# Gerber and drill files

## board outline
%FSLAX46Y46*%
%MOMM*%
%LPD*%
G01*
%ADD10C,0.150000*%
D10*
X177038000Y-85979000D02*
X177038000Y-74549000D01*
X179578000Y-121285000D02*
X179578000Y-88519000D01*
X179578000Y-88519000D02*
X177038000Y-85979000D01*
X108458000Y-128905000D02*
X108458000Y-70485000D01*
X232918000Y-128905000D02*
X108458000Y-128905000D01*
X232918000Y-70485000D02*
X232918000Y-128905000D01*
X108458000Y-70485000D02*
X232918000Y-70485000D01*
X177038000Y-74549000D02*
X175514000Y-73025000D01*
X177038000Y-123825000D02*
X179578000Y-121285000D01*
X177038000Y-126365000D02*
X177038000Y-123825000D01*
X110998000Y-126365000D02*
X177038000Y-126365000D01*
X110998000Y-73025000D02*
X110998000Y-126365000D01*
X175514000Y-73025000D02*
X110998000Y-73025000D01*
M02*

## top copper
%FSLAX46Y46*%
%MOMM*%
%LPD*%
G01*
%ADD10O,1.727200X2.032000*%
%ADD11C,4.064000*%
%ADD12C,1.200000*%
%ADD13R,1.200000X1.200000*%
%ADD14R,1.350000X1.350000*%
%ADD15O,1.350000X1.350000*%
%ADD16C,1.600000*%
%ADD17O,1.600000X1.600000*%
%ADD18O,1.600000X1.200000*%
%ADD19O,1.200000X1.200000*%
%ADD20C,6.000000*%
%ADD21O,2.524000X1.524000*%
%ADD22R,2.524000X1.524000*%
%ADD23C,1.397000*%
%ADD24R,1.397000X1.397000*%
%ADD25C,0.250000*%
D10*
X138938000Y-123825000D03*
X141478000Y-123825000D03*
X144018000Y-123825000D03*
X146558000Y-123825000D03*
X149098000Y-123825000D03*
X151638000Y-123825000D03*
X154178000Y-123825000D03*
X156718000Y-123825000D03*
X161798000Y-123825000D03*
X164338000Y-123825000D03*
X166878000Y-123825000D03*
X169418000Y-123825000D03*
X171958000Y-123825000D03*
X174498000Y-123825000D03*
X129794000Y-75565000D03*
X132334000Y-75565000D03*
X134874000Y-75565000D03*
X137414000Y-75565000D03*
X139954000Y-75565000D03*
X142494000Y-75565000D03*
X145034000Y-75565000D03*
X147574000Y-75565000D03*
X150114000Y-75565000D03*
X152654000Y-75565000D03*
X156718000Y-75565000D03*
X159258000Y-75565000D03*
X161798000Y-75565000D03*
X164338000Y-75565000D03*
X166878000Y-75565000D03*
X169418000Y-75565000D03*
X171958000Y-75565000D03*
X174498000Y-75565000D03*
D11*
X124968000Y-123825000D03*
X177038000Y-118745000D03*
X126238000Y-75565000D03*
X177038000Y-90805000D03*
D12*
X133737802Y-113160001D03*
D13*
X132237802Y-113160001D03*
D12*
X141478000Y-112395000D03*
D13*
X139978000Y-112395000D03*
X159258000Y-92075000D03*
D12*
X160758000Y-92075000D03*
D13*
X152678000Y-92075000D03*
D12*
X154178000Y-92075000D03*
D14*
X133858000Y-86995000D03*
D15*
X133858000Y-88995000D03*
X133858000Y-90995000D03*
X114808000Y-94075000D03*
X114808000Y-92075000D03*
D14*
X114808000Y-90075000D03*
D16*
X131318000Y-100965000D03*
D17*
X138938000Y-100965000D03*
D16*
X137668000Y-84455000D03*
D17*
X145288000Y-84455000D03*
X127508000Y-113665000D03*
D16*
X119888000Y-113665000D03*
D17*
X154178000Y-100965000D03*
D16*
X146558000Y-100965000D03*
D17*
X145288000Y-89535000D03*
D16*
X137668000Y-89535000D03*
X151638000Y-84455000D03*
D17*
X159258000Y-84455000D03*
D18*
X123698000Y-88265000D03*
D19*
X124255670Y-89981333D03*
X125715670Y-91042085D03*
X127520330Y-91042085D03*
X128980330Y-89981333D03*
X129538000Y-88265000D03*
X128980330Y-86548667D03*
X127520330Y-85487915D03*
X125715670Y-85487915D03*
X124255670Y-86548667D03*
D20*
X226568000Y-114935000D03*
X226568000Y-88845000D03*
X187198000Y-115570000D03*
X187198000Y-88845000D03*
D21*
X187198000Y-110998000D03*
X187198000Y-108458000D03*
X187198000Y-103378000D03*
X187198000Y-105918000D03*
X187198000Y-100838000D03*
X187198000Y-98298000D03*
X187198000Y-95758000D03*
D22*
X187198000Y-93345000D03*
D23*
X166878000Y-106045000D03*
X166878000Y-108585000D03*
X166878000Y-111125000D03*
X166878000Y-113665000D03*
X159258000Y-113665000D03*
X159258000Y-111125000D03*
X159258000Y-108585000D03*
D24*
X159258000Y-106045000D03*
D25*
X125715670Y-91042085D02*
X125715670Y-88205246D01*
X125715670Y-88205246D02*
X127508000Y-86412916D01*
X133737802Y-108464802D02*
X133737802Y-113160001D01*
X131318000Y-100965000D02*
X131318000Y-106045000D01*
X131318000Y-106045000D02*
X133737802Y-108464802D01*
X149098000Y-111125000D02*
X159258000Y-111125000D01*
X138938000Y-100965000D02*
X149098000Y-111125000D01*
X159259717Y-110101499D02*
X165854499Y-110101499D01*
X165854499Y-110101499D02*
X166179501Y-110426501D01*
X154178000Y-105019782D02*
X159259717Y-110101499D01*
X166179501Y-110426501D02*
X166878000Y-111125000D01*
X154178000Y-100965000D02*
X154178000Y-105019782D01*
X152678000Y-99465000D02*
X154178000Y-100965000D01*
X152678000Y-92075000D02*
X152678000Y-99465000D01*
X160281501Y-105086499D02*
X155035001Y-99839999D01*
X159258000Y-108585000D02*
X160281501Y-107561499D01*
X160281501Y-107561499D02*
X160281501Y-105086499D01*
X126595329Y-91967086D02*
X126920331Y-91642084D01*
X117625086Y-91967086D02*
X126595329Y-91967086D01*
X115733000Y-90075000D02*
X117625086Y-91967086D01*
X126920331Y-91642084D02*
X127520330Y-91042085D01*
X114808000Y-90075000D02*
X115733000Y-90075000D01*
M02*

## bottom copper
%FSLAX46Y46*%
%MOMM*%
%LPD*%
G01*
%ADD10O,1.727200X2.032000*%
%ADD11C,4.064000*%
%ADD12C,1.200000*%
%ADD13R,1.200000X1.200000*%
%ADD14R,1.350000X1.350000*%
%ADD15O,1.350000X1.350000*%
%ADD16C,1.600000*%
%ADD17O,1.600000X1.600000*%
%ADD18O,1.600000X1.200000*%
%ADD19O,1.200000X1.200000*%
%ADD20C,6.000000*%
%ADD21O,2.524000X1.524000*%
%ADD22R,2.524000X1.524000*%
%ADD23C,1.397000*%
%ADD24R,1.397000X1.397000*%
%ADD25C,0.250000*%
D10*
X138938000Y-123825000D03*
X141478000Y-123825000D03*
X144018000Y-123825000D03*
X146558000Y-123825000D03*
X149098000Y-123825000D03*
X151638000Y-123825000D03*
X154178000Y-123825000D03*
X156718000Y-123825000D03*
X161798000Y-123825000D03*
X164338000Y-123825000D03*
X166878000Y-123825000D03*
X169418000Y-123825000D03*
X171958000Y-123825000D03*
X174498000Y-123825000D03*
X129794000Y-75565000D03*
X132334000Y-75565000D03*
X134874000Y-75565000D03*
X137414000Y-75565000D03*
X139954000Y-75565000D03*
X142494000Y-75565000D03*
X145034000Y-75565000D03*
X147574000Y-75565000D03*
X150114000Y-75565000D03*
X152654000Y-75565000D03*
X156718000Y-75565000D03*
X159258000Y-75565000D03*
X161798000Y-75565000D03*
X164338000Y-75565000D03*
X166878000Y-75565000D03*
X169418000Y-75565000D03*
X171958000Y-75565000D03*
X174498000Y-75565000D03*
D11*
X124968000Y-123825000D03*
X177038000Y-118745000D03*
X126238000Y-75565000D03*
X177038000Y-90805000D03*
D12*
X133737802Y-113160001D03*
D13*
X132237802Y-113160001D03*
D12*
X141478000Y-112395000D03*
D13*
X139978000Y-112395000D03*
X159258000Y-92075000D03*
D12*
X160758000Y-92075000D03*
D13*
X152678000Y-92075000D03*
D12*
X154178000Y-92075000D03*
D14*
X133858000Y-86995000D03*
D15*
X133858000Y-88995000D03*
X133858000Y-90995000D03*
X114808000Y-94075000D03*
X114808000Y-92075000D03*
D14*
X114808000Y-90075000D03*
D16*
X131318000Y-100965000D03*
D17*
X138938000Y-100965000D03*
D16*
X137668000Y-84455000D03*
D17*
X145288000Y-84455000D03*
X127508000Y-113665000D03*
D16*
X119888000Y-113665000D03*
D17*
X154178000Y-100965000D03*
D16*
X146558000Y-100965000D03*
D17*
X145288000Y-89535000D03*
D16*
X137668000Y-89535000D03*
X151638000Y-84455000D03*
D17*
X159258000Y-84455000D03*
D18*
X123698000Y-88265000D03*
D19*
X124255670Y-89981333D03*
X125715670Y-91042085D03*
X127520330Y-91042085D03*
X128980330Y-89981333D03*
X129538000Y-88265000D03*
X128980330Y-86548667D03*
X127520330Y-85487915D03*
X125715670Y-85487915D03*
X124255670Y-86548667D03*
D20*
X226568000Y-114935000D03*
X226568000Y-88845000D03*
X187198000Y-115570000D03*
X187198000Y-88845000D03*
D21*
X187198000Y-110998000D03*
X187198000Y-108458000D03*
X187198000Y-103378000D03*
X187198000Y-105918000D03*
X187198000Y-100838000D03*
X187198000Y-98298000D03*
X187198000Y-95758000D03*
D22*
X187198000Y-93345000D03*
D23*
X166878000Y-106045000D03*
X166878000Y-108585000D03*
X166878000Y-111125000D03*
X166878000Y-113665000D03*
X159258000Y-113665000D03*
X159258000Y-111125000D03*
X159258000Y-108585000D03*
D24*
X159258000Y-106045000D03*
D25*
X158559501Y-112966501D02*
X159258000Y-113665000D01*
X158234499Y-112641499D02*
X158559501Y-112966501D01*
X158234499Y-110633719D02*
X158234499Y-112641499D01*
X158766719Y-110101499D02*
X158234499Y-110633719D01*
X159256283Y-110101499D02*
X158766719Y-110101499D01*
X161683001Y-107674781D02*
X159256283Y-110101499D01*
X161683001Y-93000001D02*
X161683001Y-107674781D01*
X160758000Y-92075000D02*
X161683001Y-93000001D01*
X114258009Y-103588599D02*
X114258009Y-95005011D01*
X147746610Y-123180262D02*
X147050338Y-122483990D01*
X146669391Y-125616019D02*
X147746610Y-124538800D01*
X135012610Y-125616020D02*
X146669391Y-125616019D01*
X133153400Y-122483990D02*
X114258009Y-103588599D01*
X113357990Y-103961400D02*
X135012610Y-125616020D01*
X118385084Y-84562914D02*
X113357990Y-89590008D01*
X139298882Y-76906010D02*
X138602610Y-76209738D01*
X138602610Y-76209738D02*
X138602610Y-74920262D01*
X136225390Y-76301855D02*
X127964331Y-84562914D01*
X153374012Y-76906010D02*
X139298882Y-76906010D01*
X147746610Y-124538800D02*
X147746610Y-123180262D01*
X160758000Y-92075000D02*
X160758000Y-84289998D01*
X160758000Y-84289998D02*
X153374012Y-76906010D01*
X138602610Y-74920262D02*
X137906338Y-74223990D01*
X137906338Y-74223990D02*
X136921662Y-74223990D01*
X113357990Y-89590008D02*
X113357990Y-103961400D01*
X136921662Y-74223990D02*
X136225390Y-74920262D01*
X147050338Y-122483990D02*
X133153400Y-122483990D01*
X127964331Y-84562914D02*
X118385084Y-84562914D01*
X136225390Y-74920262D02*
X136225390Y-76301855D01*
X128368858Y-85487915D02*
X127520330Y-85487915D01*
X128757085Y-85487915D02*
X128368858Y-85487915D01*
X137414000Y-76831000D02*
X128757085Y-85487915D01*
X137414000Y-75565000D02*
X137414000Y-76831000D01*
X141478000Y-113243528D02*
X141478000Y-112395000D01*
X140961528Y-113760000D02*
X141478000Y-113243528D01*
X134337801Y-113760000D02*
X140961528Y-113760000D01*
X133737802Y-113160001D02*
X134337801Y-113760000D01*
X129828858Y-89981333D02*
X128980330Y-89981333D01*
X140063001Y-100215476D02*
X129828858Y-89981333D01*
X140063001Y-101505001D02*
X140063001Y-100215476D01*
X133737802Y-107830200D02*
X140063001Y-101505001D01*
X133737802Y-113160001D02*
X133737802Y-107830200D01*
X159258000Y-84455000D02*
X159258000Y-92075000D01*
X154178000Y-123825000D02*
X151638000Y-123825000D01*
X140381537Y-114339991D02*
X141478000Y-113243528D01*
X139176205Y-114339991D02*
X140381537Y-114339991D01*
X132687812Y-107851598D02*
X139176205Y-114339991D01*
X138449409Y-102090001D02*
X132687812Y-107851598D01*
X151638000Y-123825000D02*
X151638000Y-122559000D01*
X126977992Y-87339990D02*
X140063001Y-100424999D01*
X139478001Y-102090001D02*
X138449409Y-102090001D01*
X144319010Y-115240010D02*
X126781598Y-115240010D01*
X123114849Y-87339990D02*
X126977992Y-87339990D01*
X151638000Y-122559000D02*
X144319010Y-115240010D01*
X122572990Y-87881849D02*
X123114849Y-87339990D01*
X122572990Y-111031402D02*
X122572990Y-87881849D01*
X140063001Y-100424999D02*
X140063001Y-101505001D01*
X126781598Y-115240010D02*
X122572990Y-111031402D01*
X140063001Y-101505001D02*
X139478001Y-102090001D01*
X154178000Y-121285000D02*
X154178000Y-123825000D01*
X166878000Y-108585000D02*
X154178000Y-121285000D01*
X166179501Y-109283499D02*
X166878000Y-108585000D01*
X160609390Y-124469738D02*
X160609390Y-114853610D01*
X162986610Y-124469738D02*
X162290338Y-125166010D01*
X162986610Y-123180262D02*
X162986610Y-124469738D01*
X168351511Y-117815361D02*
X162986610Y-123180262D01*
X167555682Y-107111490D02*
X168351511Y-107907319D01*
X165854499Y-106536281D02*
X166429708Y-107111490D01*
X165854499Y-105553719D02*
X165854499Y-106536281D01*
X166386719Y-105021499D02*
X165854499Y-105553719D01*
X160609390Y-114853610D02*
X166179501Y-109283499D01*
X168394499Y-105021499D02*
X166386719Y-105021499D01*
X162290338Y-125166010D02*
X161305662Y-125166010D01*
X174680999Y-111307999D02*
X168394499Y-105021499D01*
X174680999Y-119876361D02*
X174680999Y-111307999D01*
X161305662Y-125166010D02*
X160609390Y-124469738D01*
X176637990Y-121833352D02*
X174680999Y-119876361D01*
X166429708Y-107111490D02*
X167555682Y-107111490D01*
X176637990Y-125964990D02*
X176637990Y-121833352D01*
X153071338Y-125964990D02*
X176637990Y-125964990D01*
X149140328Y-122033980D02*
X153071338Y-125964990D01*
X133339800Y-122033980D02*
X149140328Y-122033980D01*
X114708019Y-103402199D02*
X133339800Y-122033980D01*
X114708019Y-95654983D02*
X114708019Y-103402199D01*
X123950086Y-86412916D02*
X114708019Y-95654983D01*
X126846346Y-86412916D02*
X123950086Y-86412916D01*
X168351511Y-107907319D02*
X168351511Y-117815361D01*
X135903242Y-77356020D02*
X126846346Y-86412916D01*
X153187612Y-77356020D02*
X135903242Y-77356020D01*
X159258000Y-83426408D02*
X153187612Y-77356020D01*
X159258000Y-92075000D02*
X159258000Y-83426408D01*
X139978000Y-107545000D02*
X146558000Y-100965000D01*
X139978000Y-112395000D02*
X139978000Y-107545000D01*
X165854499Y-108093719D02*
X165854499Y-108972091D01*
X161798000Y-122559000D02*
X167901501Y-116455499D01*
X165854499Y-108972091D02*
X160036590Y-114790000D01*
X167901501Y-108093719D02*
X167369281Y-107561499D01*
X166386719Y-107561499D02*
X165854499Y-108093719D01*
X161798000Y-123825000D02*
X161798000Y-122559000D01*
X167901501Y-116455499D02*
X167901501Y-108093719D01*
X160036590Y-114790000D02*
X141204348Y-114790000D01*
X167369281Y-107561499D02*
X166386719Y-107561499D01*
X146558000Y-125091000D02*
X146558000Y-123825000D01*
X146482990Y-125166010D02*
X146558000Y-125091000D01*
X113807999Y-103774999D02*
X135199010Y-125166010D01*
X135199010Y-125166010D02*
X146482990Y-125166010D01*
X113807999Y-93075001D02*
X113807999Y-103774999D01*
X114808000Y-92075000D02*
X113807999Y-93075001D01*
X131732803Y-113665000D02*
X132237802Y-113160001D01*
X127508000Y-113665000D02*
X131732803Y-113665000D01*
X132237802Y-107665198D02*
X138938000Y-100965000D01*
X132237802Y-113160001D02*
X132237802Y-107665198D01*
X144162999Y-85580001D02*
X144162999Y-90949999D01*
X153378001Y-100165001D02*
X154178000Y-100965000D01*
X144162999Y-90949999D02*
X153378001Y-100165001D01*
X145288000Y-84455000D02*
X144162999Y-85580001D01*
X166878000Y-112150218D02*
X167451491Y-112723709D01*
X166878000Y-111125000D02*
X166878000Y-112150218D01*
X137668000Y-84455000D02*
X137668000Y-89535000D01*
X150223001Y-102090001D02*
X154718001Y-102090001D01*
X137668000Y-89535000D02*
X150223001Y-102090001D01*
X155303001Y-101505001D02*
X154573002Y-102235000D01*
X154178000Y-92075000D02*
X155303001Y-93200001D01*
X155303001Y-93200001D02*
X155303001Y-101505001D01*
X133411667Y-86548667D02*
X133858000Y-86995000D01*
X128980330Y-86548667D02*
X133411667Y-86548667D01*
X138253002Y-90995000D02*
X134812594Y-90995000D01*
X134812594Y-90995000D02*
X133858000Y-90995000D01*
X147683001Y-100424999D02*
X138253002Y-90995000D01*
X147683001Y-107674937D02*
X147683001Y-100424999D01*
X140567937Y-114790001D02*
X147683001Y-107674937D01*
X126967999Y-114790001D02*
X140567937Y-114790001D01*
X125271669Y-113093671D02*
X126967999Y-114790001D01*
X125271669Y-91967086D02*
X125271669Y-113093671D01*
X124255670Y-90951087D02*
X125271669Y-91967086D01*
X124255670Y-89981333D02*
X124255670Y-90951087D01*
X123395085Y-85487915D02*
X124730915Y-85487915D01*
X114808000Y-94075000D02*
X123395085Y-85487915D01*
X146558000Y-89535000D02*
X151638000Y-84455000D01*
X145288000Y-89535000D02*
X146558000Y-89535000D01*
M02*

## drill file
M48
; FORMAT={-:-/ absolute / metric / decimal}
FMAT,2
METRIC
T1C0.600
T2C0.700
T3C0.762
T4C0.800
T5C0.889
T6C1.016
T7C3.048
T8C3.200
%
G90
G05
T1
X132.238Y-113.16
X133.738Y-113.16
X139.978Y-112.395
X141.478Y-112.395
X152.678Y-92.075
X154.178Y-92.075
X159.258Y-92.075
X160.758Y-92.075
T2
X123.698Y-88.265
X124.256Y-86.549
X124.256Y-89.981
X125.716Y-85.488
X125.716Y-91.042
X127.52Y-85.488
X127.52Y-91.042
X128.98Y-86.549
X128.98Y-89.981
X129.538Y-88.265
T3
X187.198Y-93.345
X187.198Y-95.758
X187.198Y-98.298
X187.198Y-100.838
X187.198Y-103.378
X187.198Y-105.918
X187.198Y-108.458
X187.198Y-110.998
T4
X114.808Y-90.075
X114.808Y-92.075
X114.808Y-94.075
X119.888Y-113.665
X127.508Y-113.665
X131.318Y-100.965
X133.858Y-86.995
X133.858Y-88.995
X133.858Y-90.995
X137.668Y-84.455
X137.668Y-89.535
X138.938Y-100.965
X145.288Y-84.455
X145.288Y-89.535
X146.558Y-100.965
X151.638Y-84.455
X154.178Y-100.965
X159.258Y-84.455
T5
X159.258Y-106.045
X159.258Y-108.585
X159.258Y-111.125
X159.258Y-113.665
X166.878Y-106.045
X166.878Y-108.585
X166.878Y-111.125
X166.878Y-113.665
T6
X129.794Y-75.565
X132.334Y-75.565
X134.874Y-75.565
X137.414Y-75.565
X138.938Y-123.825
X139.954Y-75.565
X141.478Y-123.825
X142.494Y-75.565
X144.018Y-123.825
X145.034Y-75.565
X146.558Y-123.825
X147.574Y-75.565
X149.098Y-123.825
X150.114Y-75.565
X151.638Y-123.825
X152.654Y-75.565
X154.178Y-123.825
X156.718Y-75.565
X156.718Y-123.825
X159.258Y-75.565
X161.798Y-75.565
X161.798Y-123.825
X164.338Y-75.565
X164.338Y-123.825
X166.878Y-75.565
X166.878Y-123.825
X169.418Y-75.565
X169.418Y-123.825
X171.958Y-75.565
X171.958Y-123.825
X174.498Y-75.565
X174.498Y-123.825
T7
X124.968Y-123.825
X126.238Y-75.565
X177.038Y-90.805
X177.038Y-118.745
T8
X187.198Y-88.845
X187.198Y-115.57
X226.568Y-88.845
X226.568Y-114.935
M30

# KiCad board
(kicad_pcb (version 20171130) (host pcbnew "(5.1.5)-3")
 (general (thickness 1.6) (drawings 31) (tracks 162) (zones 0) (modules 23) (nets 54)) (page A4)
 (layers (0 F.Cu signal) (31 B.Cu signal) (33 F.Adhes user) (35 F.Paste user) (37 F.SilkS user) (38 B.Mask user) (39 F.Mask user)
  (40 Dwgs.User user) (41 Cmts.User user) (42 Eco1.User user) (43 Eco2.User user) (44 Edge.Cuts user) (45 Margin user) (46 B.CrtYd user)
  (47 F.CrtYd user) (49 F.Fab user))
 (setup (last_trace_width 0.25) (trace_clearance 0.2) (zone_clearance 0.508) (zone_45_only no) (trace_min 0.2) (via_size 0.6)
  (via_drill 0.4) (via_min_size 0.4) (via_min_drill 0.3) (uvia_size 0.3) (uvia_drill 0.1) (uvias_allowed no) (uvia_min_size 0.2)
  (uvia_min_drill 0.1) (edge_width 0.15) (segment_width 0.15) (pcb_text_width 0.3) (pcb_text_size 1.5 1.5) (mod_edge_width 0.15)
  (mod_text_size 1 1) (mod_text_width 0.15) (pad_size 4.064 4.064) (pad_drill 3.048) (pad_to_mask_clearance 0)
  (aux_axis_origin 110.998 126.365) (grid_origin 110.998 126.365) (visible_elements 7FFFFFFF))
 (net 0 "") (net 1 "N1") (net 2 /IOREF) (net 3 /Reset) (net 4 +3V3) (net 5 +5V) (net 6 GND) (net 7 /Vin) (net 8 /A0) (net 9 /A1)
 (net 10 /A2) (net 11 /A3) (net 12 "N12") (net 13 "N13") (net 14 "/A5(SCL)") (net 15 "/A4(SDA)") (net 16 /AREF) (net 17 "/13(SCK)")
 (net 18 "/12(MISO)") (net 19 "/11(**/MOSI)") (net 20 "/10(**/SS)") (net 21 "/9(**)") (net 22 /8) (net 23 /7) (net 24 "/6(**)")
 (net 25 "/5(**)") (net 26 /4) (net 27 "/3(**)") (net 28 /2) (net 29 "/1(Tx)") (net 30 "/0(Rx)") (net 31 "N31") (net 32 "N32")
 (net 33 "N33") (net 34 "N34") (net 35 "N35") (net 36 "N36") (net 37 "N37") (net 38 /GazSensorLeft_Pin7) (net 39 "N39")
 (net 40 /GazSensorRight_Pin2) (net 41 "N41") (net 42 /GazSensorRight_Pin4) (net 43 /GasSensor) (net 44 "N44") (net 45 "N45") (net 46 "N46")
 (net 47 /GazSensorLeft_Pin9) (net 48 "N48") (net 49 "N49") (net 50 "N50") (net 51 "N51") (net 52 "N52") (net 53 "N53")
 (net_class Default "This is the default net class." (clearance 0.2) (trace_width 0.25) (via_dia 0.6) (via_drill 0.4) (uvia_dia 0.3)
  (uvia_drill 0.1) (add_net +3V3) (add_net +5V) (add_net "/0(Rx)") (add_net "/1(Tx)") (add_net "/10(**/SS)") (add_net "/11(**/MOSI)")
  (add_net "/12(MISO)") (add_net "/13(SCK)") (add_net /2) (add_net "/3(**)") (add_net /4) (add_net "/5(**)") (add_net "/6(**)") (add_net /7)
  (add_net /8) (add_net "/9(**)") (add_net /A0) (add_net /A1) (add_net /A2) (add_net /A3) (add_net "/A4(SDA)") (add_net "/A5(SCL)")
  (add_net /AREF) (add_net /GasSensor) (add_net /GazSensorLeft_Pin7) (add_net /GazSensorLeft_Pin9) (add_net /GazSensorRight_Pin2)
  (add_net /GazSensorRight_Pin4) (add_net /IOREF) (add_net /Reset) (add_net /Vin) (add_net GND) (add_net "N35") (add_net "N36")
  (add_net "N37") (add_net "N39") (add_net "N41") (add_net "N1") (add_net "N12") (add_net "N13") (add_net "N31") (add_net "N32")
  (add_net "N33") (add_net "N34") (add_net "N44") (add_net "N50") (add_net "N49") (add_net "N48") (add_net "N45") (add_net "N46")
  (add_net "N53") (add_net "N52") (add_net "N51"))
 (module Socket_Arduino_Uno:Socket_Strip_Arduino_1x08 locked (layer F.Cu) (at 138.938 123.825)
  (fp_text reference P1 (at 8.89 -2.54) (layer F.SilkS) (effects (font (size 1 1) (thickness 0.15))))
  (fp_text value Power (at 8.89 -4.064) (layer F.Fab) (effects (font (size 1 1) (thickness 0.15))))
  (pad 1 thru_hole oval (at 0 0) (size 1.7272 2.032) (drill 1.016) (layers *.Cu *.Mask F.SilkS) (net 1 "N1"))
  (pad 2 thru_hole oval (at 2.54 0) (size 1.7272 2.032) (drill 1.016) (layers *.Cu *.Mask F.SilkS) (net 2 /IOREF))
  (pad 3 thru_hole oval (at 5.08 0) (size 1.7272 2.032) (drill 1.016) (layers *.Cu *.Mask F.SilkS) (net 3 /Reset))
  (pad 4 thru_hole oval (at 7.62 0) (size 1.7272 2.032) (drill 1.016) (layers *.Cu *.Mask F.SilkS) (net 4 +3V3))
  (pad 5 thru_hole oval (at 10.16 0) (size 1.7272 2.032) (drill 1.016) (layers *.Cu *.Mask F.SilkS) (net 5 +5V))
  (pad 6 thru_hole oval (at 12.7 0) (size 1.7272 2.032) (drill 1.016) (layers *.Cu *.Mask F.SilkS) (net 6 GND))
  (pad 7 thru_hole oval (at 15.24 0) (size 1.7272 2.032) (drill 1.016) (layers *.Cu *.Mask F.SilkS) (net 6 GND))
  (pad 8 thru_hole oval (at 17.78 0) (size 1.7272 2.032) (drill 1.016) (layers *.Cu *.Mask F.SilkS) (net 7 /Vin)))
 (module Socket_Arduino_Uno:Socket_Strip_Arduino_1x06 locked (layer F.Cu) (at 161.798 123.825)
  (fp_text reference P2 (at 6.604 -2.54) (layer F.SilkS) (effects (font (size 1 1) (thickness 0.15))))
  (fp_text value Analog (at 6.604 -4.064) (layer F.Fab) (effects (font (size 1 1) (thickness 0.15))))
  (pad 1 thru_hole oval (at 0 0) (size 1.7272 2.032) (drill 1.016) (layers *.Cu *.Mask F.SilkS) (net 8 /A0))
  (pad 2 thru_hole oval (at 2.54 0) (size 1.7272 2.032) (drill 1.016) (layers *.Cu *.Mask F.SilkS) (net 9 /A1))
  (pad 3 thru_hole oval (at 5.08 0) (size 1.7272 2.032) (drill 1.016) (layers *.Cu *.Mask F.SilkS) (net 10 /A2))
  (pad 4 thru_hole oval (at 7.62 0) (size 1.7272 2.032) (drill 1.016) (layers *.Cu *.Mask F.SilkS) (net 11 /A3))
  (pad 5 thru_hole oval (at 10.16 0) (size 1.7272 2.032) (drill 1.016) (layers *.Cu *.Mask F.SilkS) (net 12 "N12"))
  (pad 6 thru_hole oval (at 12.7 0) (size 1.7272 2.032) (drill 1.016) (layers *.Cu *.Mask F.SilkS) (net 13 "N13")))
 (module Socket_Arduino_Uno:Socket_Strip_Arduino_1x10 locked (layer F.Cu) (at 129.794 75.565)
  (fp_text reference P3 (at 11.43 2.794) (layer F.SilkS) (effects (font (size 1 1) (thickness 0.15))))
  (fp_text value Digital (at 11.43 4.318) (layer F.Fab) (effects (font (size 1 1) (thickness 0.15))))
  (pad 1 thru_hole oval (at 0 0) (size 1.7272 2.032) (drill 1.016) (layers *.Cu *.Mask F.SilkS) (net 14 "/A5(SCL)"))
  (pad 2 thru_hole oval (at 2.54 0) (size 1.7272 2.032) (drill 1.016) (layers *.Cu *.Mask F.SilkS) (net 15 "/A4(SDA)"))
  (pad 3 thru_hole oval (at 5.08 0) (size 1.7272 2.032) (drill 1.016) (layers *.Cu *.Mask F.SilkS) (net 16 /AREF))
  (pad 4 thru_hole oval (at 7.62 0) (size 1.7272 2.032) (drill 1.016) (layers *.Cu *.Mask F.SilkS) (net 6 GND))
  (pad 5 thru_hole oval (at 10.16 0) (size 1.7272 2.032) (drill 1.016) (layers *.Cu *.Mask F.SilkS) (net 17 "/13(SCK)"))
  (pad 6 thru_hole oval (at 12.7 0) (size 1.7272 2.032) (drill 1.016) (layers *.Cu *.Mask F.SilkS) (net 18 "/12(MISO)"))
  (pad 7 thru_hole oval (at 15.24 0) (size 1.7272 2.032) (drill 1.016) (layers *.Cu *.Mask F.SilkS) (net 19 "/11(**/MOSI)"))
  (pad 8 thru_hole oval (at 17.78 0) (size 1.7272 2.032) (drill 1.016) (layers *.Cu *.Mask F.SilkS) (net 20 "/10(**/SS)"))
  (pad 9 thru_hole oval (at 20.32 0) (size 1.7272 2.032) (drill 1.016) (layers *.Cu *.Mask F.SilkS) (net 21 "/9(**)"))
  (pad 10 thru_hole oval (at 22.86 0) (size 1.7272 2.032) (drill 1.016) (layers *.Cu *.Mask F.SilkS) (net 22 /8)))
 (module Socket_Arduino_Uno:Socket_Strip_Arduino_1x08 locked (layer F.Cu) (at 156.718 75.565)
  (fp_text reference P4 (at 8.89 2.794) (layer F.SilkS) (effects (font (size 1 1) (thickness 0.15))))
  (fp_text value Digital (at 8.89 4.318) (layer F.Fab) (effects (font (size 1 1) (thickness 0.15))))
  (pad 1 thru_hole oval (at 0 0) (size 1.7272 2.032) (drill 1.016) (layers *.Cu *.Mask F.SilkS) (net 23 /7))
  (pad 2 thru_hole oval (at 2.54 0) (size 1.7272 2.032) (drill 1.016) (layers *.Cu *.Mask F.SilkS) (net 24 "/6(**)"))
  (pad 3 thru_hole oval (at 5.08 0) (size 1.7272 2.032) (drill 1.016) (layers *.Cu *.Mask F.SilkS) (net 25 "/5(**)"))
  (pad 4 thru_hole oval (at 7.62 0) (size 1.7272 2.032) (drill 1.016) (layers *.Cu *.Mask F.SilkS) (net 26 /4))
  (pad 5 thru_hole oval (at 10.16 0) (size 1.7272 2.032) (drill 1.016) (layers *.Cu *.Mask F.SilkS) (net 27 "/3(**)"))
  (pad 6 thru_hole oval (at 12.7 0) (size 1.7272 2.032) (drill 1.016) (layers *.Cu *.Mask F.SilkS) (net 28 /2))
  (pad 7 thru_hole oval (at 15.24 0) (size 1.7272 2.032) (drill 1.016) (layers *.Cu *.Mask F.SilkS) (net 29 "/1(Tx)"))
  (pad 8 thru_hole oval (at 17.78 0) (size 1.7272 2.032) (drill 1.016) (layers *.Cu *.Mask F.SilkS) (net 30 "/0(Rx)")))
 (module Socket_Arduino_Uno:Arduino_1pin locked (layer F.Cu) (at 124.968 123.825)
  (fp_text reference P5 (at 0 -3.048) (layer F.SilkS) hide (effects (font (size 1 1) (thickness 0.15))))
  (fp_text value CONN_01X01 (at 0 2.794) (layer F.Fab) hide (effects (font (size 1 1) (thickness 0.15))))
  (pad 1 thru_hole circle (at 0 0) (size 4.064 4.064) (drill 3.048) (layers *.Cu *.Mask F.SilkS) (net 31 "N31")))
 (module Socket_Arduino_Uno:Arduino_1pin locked (layer F.Cu) (at 177.038 118.745)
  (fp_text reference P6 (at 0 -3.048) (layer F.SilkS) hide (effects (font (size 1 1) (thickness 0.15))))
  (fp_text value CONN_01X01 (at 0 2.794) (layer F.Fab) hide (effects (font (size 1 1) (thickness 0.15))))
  (pad 1 thru_hole circle (at 0 0) (size 4.064 4.064) (drill 3.048) (layers *.Cu *.Mask F.SilkS) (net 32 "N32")))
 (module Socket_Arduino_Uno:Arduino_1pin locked (layer F.Cu) (at 126.238 75.565)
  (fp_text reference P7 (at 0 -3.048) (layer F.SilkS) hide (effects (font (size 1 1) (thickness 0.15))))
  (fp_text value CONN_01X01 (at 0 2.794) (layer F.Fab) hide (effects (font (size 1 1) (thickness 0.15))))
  (pad 1 thru_hole circle (at 0 0) (size 4.064 4.064) (drill 3.048) (layers *.Cu *.Mask F.SilkS) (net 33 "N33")))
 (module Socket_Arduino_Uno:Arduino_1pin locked (layer F.Cu) (at 177.038 90.805)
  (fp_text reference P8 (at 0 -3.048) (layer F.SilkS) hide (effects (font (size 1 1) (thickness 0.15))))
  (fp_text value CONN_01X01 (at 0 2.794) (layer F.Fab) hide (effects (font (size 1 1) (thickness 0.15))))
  (pad 1 thru_hole circle (at 0 0) (size 4.064 4.064) (drill 3.048) (layers *.Cu *.Mask F.SilkS) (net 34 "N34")))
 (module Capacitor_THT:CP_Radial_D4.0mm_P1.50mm (layer F.Cu) (at 132.237802 113.160001)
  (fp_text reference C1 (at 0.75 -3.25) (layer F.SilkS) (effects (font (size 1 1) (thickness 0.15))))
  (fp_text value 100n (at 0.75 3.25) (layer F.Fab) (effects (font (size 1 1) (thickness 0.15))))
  (pad 2 thru_hole circle (at 1.5 0) (size 1.2 1.2) (drill 0.6) (layers *.Cu *.Mask) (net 6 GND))
  (pad 1 thru_hole rect (at 0 0) (size 1.2 1.2) (drill 0.6) (layers *.Cu *.Mask) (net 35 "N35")))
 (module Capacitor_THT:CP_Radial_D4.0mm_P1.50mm (layer F.Cu) (at 139.978 112.395)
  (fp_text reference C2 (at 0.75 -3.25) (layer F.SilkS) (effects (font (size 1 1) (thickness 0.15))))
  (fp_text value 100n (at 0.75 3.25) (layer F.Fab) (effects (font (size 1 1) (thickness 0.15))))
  (pad 2 thru_hole circle (at 1.5 0) (size 1.2 1.2) (drill 0.6) (layers *.Cu *.Mask) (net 6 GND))
  (pad 1 thru_hole rect (at 0 0) (size 1.2 1.2) (drill 0.6) (layers *.Cu *.Mask) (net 8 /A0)))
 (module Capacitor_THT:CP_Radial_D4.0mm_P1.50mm (layer F.Cu) (at 159.258 92.075)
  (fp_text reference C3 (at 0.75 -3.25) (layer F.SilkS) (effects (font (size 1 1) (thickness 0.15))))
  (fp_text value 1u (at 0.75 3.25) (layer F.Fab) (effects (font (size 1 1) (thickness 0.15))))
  (pad 1 thru_hole rect (at 0 0) (size 1.2 1.2) (drill 0.6) (layers *.Cu *.Mask) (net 6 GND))
  (pad 2 thru_hole circle (at 1.5 0) (size 1.2 1.2) (drill 0.6) (layers *.Cu *.Mask) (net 5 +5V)))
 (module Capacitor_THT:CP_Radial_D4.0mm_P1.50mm (layer F.Cu) (at 152.678 92.075)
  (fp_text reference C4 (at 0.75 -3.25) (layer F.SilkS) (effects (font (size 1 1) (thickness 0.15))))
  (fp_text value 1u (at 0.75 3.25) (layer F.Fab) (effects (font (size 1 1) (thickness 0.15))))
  (pad 1 thru_hole rect (at 0 0) (size 1.2 1.2) (drill 0.6) (layers *.Cu *.Mask) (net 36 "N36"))
  (pad 2 thru_hole circle (at 1.5 0) (size 1.2 1.2) (drill 0.6) (layers *.Cu *.Mask) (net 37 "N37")))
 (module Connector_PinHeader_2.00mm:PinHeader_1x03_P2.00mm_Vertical (layer F.Cu) (at 133.858 86.995)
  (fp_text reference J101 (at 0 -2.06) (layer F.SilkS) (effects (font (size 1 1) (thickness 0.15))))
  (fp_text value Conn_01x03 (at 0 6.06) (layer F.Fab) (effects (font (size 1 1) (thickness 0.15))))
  (pad 1 thru_hole rect (at 0 0) (size 1.35 1.35) (drill 0.8) (layers *.Cu *.Mask) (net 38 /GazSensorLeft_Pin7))
  (pad 2 thru_hole oval (at 0 2) (size 1.35 1.35) (drill 0.8) (layers *.Cu *.Mask) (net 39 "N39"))
  (pad 3 thru_hole oval (at 0 4) (size 1.35 1.35) (drill 0.8) (layers *.Cu *.Mask) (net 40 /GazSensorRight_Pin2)))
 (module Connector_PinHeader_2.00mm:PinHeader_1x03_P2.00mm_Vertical (layer F.Cu) (at 114.808 90.075)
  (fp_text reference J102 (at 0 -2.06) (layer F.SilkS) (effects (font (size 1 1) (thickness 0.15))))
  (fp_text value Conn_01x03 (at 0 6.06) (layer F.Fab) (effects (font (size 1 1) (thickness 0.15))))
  (pad 3 thru_hole oval (at 0 4) (size 1.35 1.35) (drill 0.8) (layers *.Cu *.Mask) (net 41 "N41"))
  (pad 2 thru_hole oval (at 0 2) (size 1.35 1.35) (drill 0.8) (layers *.Cu *.Mask) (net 4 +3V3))
  (pad 1 thru_hole rect (at 0 0) (size 1.35 1.35) (drill 0.8) (layers *.Cu *.Mask) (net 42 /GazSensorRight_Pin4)))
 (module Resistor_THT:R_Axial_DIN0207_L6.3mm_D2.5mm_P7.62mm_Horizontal (layer F.Cu) (at 131.318 100.965)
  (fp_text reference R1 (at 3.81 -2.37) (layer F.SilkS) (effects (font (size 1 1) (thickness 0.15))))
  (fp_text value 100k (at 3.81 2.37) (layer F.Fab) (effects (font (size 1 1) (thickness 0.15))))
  (pad 1 thru_hole circle (at 0 0) (size 1.6 1.6) (drill 0.8) (layers *.Cu *.Mask) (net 6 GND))
  (pad 2 thru_hole oval (at 7.62 0) (size 1.6 1.6) (drill 0.8) (layers *.Cu *.Mask) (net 35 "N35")))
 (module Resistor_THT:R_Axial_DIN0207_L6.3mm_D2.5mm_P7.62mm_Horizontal (layer F.Cu) (at 137.668 84.455)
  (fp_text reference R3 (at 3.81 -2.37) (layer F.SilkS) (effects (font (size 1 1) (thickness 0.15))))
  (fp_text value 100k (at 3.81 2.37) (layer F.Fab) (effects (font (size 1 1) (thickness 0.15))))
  (pad 1 thru_hole circle (at 0 0) (size 1.6 1.6) (drill 0.8) (layers *.Cu *.Mask) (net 37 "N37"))
  (pad 2 thru_hole oval (at 7.62 0) (size 1.6 1.6) (drill 0.8) (layers *.Cu *.Mask) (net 36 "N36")))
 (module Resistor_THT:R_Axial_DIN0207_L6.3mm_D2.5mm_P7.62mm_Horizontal (layer F.Cu) (at 119.888 113.665)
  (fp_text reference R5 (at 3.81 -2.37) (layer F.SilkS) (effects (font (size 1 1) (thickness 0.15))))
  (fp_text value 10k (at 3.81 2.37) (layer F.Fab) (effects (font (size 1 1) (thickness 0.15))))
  (pad 2 thru_hole oval (at 7.62 0) (size 1.6 1.6) (drill 0.8) (layers *.Cu *.Mask) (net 35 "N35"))
  (pad 1 thru_hole circle (at 0 0) (size 1.6 1.6) (drill 0.8) (layers *.Cu *.Mask) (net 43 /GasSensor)))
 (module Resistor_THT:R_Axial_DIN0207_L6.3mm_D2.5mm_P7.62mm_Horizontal (layer F.Cu) (at 146.558 100.965)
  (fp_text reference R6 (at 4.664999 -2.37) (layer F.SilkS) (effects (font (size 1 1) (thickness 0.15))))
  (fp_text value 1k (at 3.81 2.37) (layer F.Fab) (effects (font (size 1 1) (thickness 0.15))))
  (pad 2 thru_hole oval (at 7.62 0) (size 1.6 1.6) (drill 0.8) (layers *.Cu *.Mask) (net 36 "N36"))
  (pad 1 thru_hole circle (at 0 0) (size 1.6 1.6) (drill 0.8) (layers *.Cu *.Mask) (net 8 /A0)))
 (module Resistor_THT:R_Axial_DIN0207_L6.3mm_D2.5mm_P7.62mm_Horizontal (layer F.Cu) (at 137.668 89.535)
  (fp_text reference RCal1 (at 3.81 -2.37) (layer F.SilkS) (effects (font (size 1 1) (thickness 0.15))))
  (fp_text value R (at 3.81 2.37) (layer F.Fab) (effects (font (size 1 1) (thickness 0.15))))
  (pad 2 thru_hole oval (at 7.62 0) (size 1.6 1.6) (drill 0.8) (layers *.Cu *.Mask) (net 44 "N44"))
  (pad 1 thru_hole circle (at 0 0) (size 1.6 1.6) (drill 0.8) (layers *.Cu *.Mask) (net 37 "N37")))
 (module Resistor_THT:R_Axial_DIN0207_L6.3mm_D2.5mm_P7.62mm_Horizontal (layer F.Cu) (at 151.638 84.455)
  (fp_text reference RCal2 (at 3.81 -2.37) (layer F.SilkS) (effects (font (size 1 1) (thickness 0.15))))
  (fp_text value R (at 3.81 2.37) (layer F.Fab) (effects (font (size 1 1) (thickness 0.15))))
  (pad 1 thru_hole circle (at 0 0) (size 1.6 1.6) (drill 0.8) (layers *.Cu *.Mask) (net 44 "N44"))
  (pad 2 thru_hole oval (at 7.62 0) (size 1.6 1.6) (drill 0.8) (layers *.Cu *.Mask) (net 6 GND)))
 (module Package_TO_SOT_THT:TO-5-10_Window (layer F.Cu) (at 123.698 88.265)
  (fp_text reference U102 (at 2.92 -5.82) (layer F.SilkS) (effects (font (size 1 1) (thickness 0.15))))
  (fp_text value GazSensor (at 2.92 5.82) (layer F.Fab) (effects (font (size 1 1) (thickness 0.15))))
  (pad 1 thru_hole oval (at 0 0) (size 1.6 1.2) (drill 0.7) (layers *.Cu *.Mask) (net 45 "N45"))
  (pad 2 thru_hole oval (at 0.55767 1.716333) (size 1.2 1.2) (drill 0.7) (layers *.Cu *.Mask) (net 40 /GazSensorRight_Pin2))
  (pad 3 thru_hole oval (at 2.01767 2.777085) (size 1.2 1.2) (drill 0.7) (layers *.Cu *.Mask) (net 5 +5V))
  (pad 4 thru_hole oval (at 3.82233 2.777085) (size 1.2 1.2) (drill 0.7) (layers *.Cu *.Mask) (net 42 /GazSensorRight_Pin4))
  (pad 5 thru_hole oval (at 5.28233 1.716333) (size 1.2 1.2) (drill 0.7) (layers *.Cu *.Mask) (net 6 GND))
  (pad 6 thru_hole oval (at 5.84 0) (size 1.2 1.2) (drill 0.7) (layers *.Cu *.Mask) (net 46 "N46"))
  (pad 7 thru_hole oval (at 5.28233 -1.716333) (size 1.2 1.2) (drill 0.7) (layers *.Cu *.Mask) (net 38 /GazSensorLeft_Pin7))
  (pad 8 thru_hole oval (at 3.82233 -2.777085) (size 1.2 1.2) (drill 0.7) (layers *.Cu *.Mask) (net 6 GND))
  (pad 9 thru_hole oval (at 2.01767 -2.777085) (size 1.2 1.2) (drill 0.7) (layers *.Cu *.Mask) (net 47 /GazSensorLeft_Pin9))
  (pad 10 thru_hole oval (at 0.55767 -1.716333) (size 1.2 1.2) (drill 0.7) (layers *.Cu *.Mask) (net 6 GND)))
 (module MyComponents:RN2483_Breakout (layer F.Cu) (at 187.198 93.345 270)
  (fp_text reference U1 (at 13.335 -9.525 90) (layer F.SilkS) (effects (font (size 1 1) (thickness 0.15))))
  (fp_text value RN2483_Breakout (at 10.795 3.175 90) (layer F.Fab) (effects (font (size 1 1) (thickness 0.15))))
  (pad "" np_thru_hole circle (at 21.59 -39.37 270) (size 6 6) (drill 3.2) (layers *.Cu *.Mask))
  (pad "" np_thru_hole circle (at -4.5 -39.37 270) (size 6 6) (drill 3.2) (layers *.Cu *.Mask))
  (pad "" np_thru_hole circle (at 22.225 0 270) (size 6 6) (drill 3.2) (layers *.Cu *.Mask))
  (pad "" np_thru_hole circle (at -4.5 0 270) (size 6 6) (drill 3.2) (layers *.Cu *.Mask))
  (pad 8 thru_hole oval (at 17.653 0 270) (size 1.524 2.524) (drill 0.762) (layers *.Cu *.Mask) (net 6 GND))
  (pad 7 thru_hole oval (at 15.113 0 270) (size 1.524 2.524) (drill 0.762) (layers *.Cu *.Mask) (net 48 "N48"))
  (pad 5 thru_hole oval (at 10.033 0 270) (size 1.524 2.524) (drill 0.762) (layers *.Cu *.Mask))
  (pad 6 thru_hole oval (at 12.573 0 270) (size 1.524 2.524) (drill 0.762) (layers *.Cu *.Mask) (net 4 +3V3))
  (pad 4 thru_hole oval (at 7.493 0 270) (size 1.524 2.524) (drill 0.762) (layers *.Cu *.Mask) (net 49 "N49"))
  (pad 3 thru_hole oval (at 4.953 0 270) (size 1.524 2.524) (drill 0.762) (layers *.Cu *.Mask) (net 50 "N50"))
  (pad 2 thru_hole oval (at 2.413 0 270) (size 1.524 2.524) (drill 0.762) (layers *.Cu *.Mask) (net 22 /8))
  (pad 1 thru_hole rect (at 0 0 270) (size 1.524 2.524) (drill 0.762) (layers *.Cu *.Mask) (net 23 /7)))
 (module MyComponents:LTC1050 (layer F.Cu) (at 166.878 113.665)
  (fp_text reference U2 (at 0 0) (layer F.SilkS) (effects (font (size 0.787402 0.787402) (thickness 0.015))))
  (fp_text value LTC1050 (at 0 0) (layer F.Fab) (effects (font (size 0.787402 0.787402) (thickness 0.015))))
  (pad 8 thru_hole circle (at 0 -7.62) (size 1.397 1.397) (drill 0.889) (layers *.Cu *.Mask) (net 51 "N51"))
  (pad 7 thru_hole circle (at 0 -5.08) (size 1.397 1.397) (drill 0.889) (layers *.Cu *.Mask) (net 5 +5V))
  (pad 6 thru_hole circle (at 0 -2.54) (size 1.397 1.397) (drill 0.889) (layers *.Cu *.Mask) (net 36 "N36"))
  (pad 5 thru_hole circle (at 0 0) (size 1.397 1.397) (drill 0.889) (layers *.Cu *.Mask) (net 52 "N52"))
  (pad 4 thru_hole circle (at -7.62 0) (size 1.397 1.397) (drill 0.889) (layers *.Cu *.Mask) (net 6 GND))
  (pad 3 thru_hole circle (at -7.62 -2.54) (size 1.397 1.397) (drill 0.889) (layers *.Cu *.Mask) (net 35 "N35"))
  (pad 2 thru_hole circle (at -7.62 -5.08) (size 1.397 1.397) (drill 0.889) (layers *.Cu *.Mask) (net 37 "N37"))
  (pad 1 thru_hole rect (at -7.62 -7.62) (size 1.397 1.397) (drill 0.889) (layers *.Cu *.Mask) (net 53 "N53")))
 (gr_line (start 177.038 85.979) (end 177.038 74.549) (angle 90) (layer Edge.Cuts) (width 0.15))
 (gr_line (start 179.578 121.285) (end 179.578 88.519) (angle 90) (layer Edge.Cuts) (width 0.15))
 (gr_line (start 179.578 88.519) (end 177.038 85.979) (angle 90) (layer Edge.Cuts) (width 0.15))
 (gr_line (start 108.458 128.905) (end 108.458 70.485) (layer Edge.Cuts) (width 0.15))
 (gr_line (start 232.918 128.905) (end 108.458 128.905) (layer Edge.Cuts) (width 0.15))
 (gr_line (start 232.918 70.485) (end 232.918 128.905) (layer Edge.Cuts) (width 0.15))
 (gr_line (start 108.458 70.485) (end 232.918 70.485) (layer Edge.Cuts) (width 0.15))
 (gr_line (start 177.038 74.549) (end 175.514 73.025) (angle 90) (layer Edge.Cuts) (width 0.15))
 (gr_line (start 177.038 123.825) (end 179.578 121.285) (angle 90) (layer Edge.Cuts) (width 0.15))
 (gr_line (start 177.038 126.365) (end 177.038 123.825) (angle 90) (layer Edge.Cuts) (width 0.15))
 (gr_line (start 110.998 126.365) (end 177.038 126.365) (angle 90) (layer Edge.Cuts) (width 0.15))
 (gr_line (start 110.998 73.025) (end 110.998 126.365) (angle 90) (layer Edge.Cuts) (width 0.15))
 (gr_line (start 175.514 73.025) (end 110.998 73.025) (angle 90) (layer Edge.Cuts) (width 0.15))
 (segment (start 158.559501 112.966501) (end 159.258 113.665) (width 0.25) (layer B.Cu) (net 5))
 (segment (start 158.234499 112.641499) (end 158.559501 112.966501) (width 0.25) (layer B.Cu) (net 5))
 (segment (start 158.234499 110.633719) (end 158.234499 112.641499) (width 0.25) (layer B.Cu) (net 5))
 (segment (start 158.766719 110.101499) (end 158.234499 110.633719) (width 0.25) (layer B.Cu) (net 5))
 (segment (start 159.256283 110.101499) (end 158.766719 110.101499) (width 0.25) (layer B.Cu) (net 5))
 (segment (start 161.683001 107.674781) (end 159.256283 110.101499) (width 0.25) (layer B.Cu) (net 5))
 (segment (start 161.683001 93.000001) (end 161.683001 107.674781) (width 0.25) (layer B.Cu) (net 5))
 (segment (start 160.758 92.075) (end 161.683001 93.000001) (width 0.25) (layer B.Cu) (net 5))
 (segment (start 114.258009 103.588599) (end 114.258009 95.005011) (width 0.25) (layer B.Cu) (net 5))
 (segment (start 147.74661 123.180262) (end 147.050338 122.48399) (width 0.25) (layer B.Cu) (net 5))
 (segment (start 146.669391 125.616019) (end 147.74661 124.5388) (width 0.25) (layer B.Cu) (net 5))
 (segment (start 135.01261 125.61602) (end 146.669391 125.616019) (width 0.25) (layer B.Cu) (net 5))
 (segment (start 133.1534 122.48399) (end 114.258009 103.588599) (width 0.25) (layer B.Cu) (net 5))
 (segment (start 113.35799 103.9614) (end 135.01261 125.61602) (width 0.25) (layer B.Cu) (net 5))
 (segment (start 118.385084 84.562914) (end 113.35799 89.590008) (width 0.25) (layer B.Cu) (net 5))
 (segment (start 139.298882 76.90601) (end 138.60261 76.209738) (width 0.25) (layer B.Cu) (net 5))
 (segment (start 138.60261 76.209738) (end 138.60261 74.920262) (width 0.25) (layer B.Cu) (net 5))
 (segment (start 136.22539 76.301855) (end 127.964331 84.562914) (width 0.25) (layer B.Cu) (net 5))
 (segment (start 153.374012 76.90601) (end 139.298882 76.90601) (width 0.25) (layer B.Cu) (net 5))
 (segment (start 147.74661 124.5388) (end 147.74661 123.180262) (width 0.25) (layer B.Cu) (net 5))
 (segment (start 160.758 92.075) (end 160.758 84.289998) (width 0.25) (layer B.Cu) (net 5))
 (segment (start 160.758 84.289998) (end 153.374012 76.90601) (width 0.25) (layer B.Cu) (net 5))
 (segment (start 138.60261 74.920262) (end 137.906338 74.22399) (width 0.25) (layer B.Cu) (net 5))
 (segment (start 137.906338 74.22399) (end 136.921662 74.22399) (width 0.25) (layer B.Cu) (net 5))
 (segment (start 113.35799 89.590008) (end 113.35799 103.9614) (width 0.25) (layer B.Cu) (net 5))
 (segment (start 136.921662 74.22399) (end 136.22539 74.920262) (width 0.25) (layer B.Cu) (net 5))
 (segment (start 147.050338 122.48399) (end 133.1534 122.48399) (width 0.25) (layer B.Cu) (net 5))
 (segment (start 127.964331 84.562914) (end 118.385084 84.562914) (width 0.25) (layer B.Cu) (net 5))
 (segment (start 136.22539 74.920262) (end 136.22539 76.301855) (width 0.25) (layer B.Cu) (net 5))
 (segment (start 125.71567 91.042085) (end 125.71567 88.205246) (width 0.25) (layer F.Cu) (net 5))
 (segment (start 125.71567 88.205246) (end 127.508 86.412916) (width 0.25) (layer F.Cu) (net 5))
 (segment (start 128.368858 85.487915) (end 127.52033 85.487915) (width 0.25) (layer B.Cu) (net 6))
 (segment (start 128.757085 85.487915) (end 128.368858 85.487915) (width 0.25) (layer B.Cu) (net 6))
 (segment (start 137.414 76.831) (end 128.757085 85.487915) (width 0.25) (layer B.Cu) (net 6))
 (segment (start 137.414 75.565) (end 137.414 76.831) (width 0.25) (layer B.Cu) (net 6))
 (segment (start 141.478 113.243528) (end 141.478 112.395) (width 0.25) (layer B.Cu) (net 6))
 (segment (start 140.961528 113.76) (end 141.478 113.243528) (width 0.25) (layer B.Cu) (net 6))
 (segment (start 134.337801 113.76) (end 140.961528 113.76) (width 0.25) (layer B.Cu) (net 6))
 (segment (start 133.737802 113.160001) (end 134.337801 113.76) (width 0.25) (layer B.Cu) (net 6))
 (segment (start 129.828858 89.981333) (end 128.98033 89.981333) (width 0.25) (layer B.Cu) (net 6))
 (segment (start 140.063001 100.215476) (end 129.828858 89.981333) (width 0.25) (layer B.Cu) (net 6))
 (segment (start 140.063001 101.505001) (end 140.063001 100.215476) (width 0.25) (layer B.Cu) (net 6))
 (segment (start 133.737802 107.8302) (end 140.063001 101.505001) (width 0.25) (layer B.Cu) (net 6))
 (segment (start 133.737802 113.160001) (end 133.737802 107.8302) (width 0.25) (layer B.Cu) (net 6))
 (segment (start 159.258 84.455) (end 159.258 92.075) (width 0.25) (layer B.Cu) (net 6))
 (segment (start 154.178 123.825) (end 151.638 123.825) (width 0.25) (layer B.Cu) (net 6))
 (segment (start 140.381537 114.339991) (end 141.478 113.243528) (width 0.25) (layer B.Cu) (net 6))
 (segment (start 139.176205 114.339991) (end 140.381537 114.339991) (width 0.25) (layer B.Cu) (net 6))
 (segment (start 132.687812 107.851598) (end 139.176205 114.339991) (width 0.25) (layer B.Cu) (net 6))
 (segment (start 138.449409 102.090001) (end 132.687812 107.851598) (width 0.25) (layer B.Cu) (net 6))
 (segment (start 151.638 123.825) (end 151.638 122.559) (width 0.25) (layer B.Cu) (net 6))
 (segment (start 126.977992 87.33999) (end 140.063001 100.424999) (width 0.25) (layer B.Cu) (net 6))
 (segment (start 139.478001 102.090001) (end 138.449409 102.090001) (width 0.25) (layer B.Cu) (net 6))
 (segment (start 144.31901 115.24001) (end 126.781598 115.24001) (width 0.25) (layer B.Cu) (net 6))
 (segment (start 123.114849 87.33999) (end 126.977992 87.33999) (width 0.25) (layer B.Cu) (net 6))
 (segment (start 151.638 122.559) (end 144.31901 115.24001) (width 0.25) (layer B.Cu) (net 6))
 (segment (start 122.57299 87.881849) (end 123.114849 87.33999) (width 0.25) (layer B.Cu) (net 6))
 (segment (start 122.57299 111.031402) (end 122.57299 87.881849) (width 0.25) (layer B.Cu) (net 6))
 (segment (start 140.063001 100.424999) (end 140.063001 101.505001) (width 0.25) (layer B.Cu) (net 6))
 (segment (start 126.781598 115.24001) (end 122.57299 111.031402) (width 0.25) (layer B.Cu) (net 6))
 (segment (start 140.063001 101.505001) (end 139.478001 102.090001) (width 0.25) (layer B.Cu) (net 6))
 (segment (start 154.178 121.285) (end 154.178 123.825) (width 0.25) (layer B.Cu) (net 6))
 (segment (start 166.878 108.585) (end 154.178 121.285) (width 0.25) (layer B.Cu) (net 6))
 (segment (start 166.179501 109.283499) (end 166.878 108.585) (width 0.25) (layer B.Cu) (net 6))
 (segment (start 160.60939 124.469738) (end 160.60939 114.85361) (width 0.25) (layer B.Cu) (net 6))
 (segment (start 162.98661 124.469738) (end 162.290338 125.16601) (width 0.25) (layer B.Cu) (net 6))
 (segment (start 162.98661 123.180262) (end 162.98661 124.469738) (width 0.25) (layer B.Cu) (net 6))
 (segment (start 168.351511 117.815361) (end 162.98661 123.180262) (width 0.25) (layer B.Cu) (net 6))
 (segment (start 167.555682 107.11149) (end 168.351511 107.907319) (width 0.25) (layer B.Cu) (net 6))
 (segment (start 165.854499 106.536281) (end 166.429708 107.11149) (width 0.25) (layer B.Cu) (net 6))
 (segment (start 165.854499 105.553719) (end 165.854499 106.536281) (width 0.25) (layer B.Cu) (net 6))
 (segment (start 166.386719 105.021499) (end 165.854499 105.553719) (width 0.25) (layer B.Cu) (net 6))
 (segment (start 160.60939 114.85361) (end 166.179501 109.283499) (width 0.25) (layer B.Cu) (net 6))
 (segment (start 168.394499 105.021499) (end 166.386719 105.021499) (width 0.25) (layer B.Cu) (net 6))
 (segment (start 162.290338 125.16601) (end 161.305662 125.16601) (width 0.25) (layer B.Cu) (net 6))
 (segment (start 174.680999 111.307999) (end 168.394499 105.021499) (width 0.25) (layer B.Cu) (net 6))
 (segment (start 174.680999 119.876361) (end 174.680999 111.307999) (width 0.25) (layer B.Cu) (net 6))
 (segment (start 161.305662 125.16601) (end 160.60939 124.469738) (width 0.25) (layer B.Cu) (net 6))
 (segment (start 176.63799 121.833352) (end 174.680999 119.876361) (width 0.25) (layer B.Cu) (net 6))
 (segment (start 166.429708 107.11149) (end 167.555682 107.11149) (width 0.25) (layer B.Cu) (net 6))
 (segment (start 176.63799 125.96499) (end 176.63799 121.833352) (width 0.25) (layer B.Cu) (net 6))
 (segment (start 153.071338 125.96499) (end 176.63799 125.96499) (width 0.25) (layer B.Cu) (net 6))
 (segment (start 149.140328 122.03398) (end 153.071338 125.96499) (width 0.25) (layer B.Cu) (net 6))
 (segment (start 133.3398 122.03398) (end 149.140328 122.03398) (width 0.25) (layer B.Cu) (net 6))
 (segment (start 114.708019 103.402199) (end 133.3398 122.03398) (width 0.25) (layer B.Cu) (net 6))
 (segment (start 114.708019 95.654983) (end 114.708019 103.402199) (width 0.25) (layer B.Cu) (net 6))
 (segment (start 123.950086 86.412916) (end 114.708019 95.654983) (width 0.25) (layer B.Cu) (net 6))
 (segment (start 126.846346 86.412916) (end 123.950086 86.412916) (width 0.25) (layer B.Cu) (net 6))
 (segment (start 168.351511 107.907319) (end 168.351511 117.815361) (width 0.25) (layer B.Cu) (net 6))
 (segment (start 135.903242 77.35602) (end 126.846346 86.412916) (width 0.25) (layer B.Cu) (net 6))
 (segment (start 153.187612 77.35602) (end 135.903242 77.35602) (width 0.25) (layer B.Cu) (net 6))
 (segment (start 159.258 83.426408) (end 153.187612 77.35602) (width 0.25) (layer B.Cu) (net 6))
 (segment (start 159.258 92.075) (end 159.258 83.426408) (width 0.25) (layer B.Cu) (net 6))
 (segment (start 133.737802 108.464802) (end 133.737802 113.160001) (width 0.25) (layer F.Cu) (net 6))
 (segment (start 131.318 100.965) (end 131.318 106.045) (width 0.25) (layer F.Cu) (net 6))
 (segment (start 131.318 106.045) (end 133.737802 108.464802) (width 0.25) (layer F.Cu) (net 6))
 (segment (start 139.978 107.545) (end 146.558 100.965) (width 0.25) (layer B.Cu) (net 8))
 (segment (start 139.978 112.395) (end 139.978 107.545) (width 0.25) (layer B.Cu) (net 8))
 (segment (start 165.854499 108.093719) (end 165.854499 108.972091) (width 0.25) (layer B.Cu) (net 8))
 (segment (start 161.798 122.559) (end 167.901501 116.455499) (width 0.25) (layer B.Cu) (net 8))
 (segment (start 165.854499 108.972091) (end 160.03659 114.79) (width 0.25) (layer B.Cu) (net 8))
 (segment (start 167.901501 108.093719) (end 167.369281 107.561499) (width 0.25) (layer B.Cu) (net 8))
 (segment (start 166.386719 107.561499) (end 165.854499 108.093719) (width 0.25) (layer B.Cu) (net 8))
 (segment (start 161.798 123.825) (end 161.798 122.559) (width 0.25) (layer B.Cu) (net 8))
 (segment (start 167.901501 116.455499) (end 167.901501 108.093719) (width 0.25) (layer B.Cu) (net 8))
 (segment (start 160.03659 114.79) (end 141.204348 114.79) (width 0.25) (layer B.Cu) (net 8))
 (segment (start 167.369281 107.561499) (end 166.386719 107.561499) (width 0.25) (layer B.Cu) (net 8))
 (segment (start 146.558 125.091) (end 146.558 123.825) (width 0.25) (layer B.Cu) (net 4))
 (segment (start 146.48299 125.16601) (end 146.558 125.091) (width 0.25) (layer B.Cu) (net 4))
 (segment (start 113.807999 103.774999) (end 135.19901 125.16601) (width 0.25) (layer B.Cu) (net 4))
 (segment (start 135.19901 125.16601) (end 146.48299 125.16601) (width 0.25) (layer B.Cu) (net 4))
 (segment (start 113.807999 93.075001) (end 113.807999 103.774999) (width 0.25) (layer B.Cu) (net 4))
 (segment (start 114.808 92.075) (end 113.807999 93.075001) (width 0.25) (layer B.Cu) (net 4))
 (segment (start 131.732803 113.665) (end 132.237802 113.160001) (width 0.25) (layer B.Cu) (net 35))
 (segment (start 127.508 113.665) (end 131.732803 113.665) (width 0.25) (layer B.Cu) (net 35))
 (segment (start 132.237802 107.665198) (end 138.938 100.965) (width 0.25) (layer B.Cu) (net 35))
 (segment (start 132.237802 113.160001) (end 132.237802 107.665198) (width 0.25) (layer B.Cu) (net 35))
 (segment (start 149.098 111.125) (end 159.258 111.125) (width 0.25) (layer F.Cu) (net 35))
 (segment (start 138.938 100.965) (end 149.098 111.125) (width 0.25) (layer F.Cu) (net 35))
 (segment (start 144.162999 85.580001) (end 144.162999 90.949999) (width 0.25) (layer B.Cu) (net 36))
 (segment (start 153.378001 100.165001) (end 154.178 100.965) (width 0.25) (layer B.Cu) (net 36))
 (segment (start 144.162999 90.949999) (end 153.378001 100.165001) (width 0.25) (layer B.Cu) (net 36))
 (segment (start 145.288 84.455) (end 144.162999 85.580001) (width 0.25) (layer B.Cu) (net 36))
 (segment (start 166.878 112.150218) (end 167.451491 112.723709) (width 0.25) (layer B.Cu) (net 36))
 (segment (start 166.878 111.125) (end 166.878 112.150218) (width 0.25) (layer B.Cu) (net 36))
 (segment (start 159.259717 110.101499) (end 165.854499 110.101499) (width 0.25) (layer F.Cu) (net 36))
 (segment (start 165.854499 110.101499) (end 166.179501 110.426501) (width 0.25) (layer F.Cu) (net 36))
 (segment (start 154.178 105.019782) (end 159.259717 110.101499) (width 0.25) (layer F.Cu) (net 36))
 (segment (start 166.179501 110.426501) (end 166.878 111.125) (width 0.25) (layer F.Cu) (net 36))
 (segment (start 154.178 100.965) (end 154.178 105.019782) (width 0.25) (layer F.Cu) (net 36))
 (segment (start 152.678 99.465) (end 154.178 100.965) (width 0.25) (layer F.Cu) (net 36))
 (segment (start 152.678 92.075) (end 152.678 99.465) (width 0.25) (layer F.Cu) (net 36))
 (segment (start 137.668 84.455) (end 137.668 89.535) (width 0.25) (layer B.Cu) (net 37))
 (segment (start 150.223001 102.090001) (end 154.718001 102.090001) (width 0.25) (layer B.Cu) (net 37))
 (segment (start 137.668 89.535) (end 150.223001 102.090001) (width 0.25) (layer B.Cu) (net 37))
 (segment (start 155.303001 101.505001) (end 154.573002 102.235) (width 0.25) (layer B.Cu) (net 37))
 (segment (start 154.178 92.075) (end 155.303001 93.200001) (width 0.25) (layer B.Cu) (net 37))
 (segment (start 155.303001 93.200001) (end 155.303001 101.505001) (width 0.25) (layer B.Cu) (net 37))
 (segment (start 160.281501 105.086499) (end 155.035001 99.839999) (width 0.25) (layer F.Cu) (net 37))
 (segment (start 159.258 108.585) (end 160.281501 107.561499) (width 0.25) (layer F.Cu) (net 37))
 (segment (start 160.281501 107.561499) (end 160.281501 105.086499) (width 0.25) (layer F.Cu) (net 37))
 (segment (start 133.411667 86.548667) (end 133.858 86.995) (width 0.25) (layer B.Cu) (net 38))
 (segment (start 128.98033 86.548667) (end 133.411667 86.548667) (width 0.25) (layer B.Cu) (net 38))
 (segment (start 138.253002 90.995) (end 134.812594 90.995) (width 0.25) (layer B.Cu) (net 40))
 (segment (start 134.812594 90.995) (end 133.858 90.995) (width 0.25) (layer B.Cu) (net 40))
 (segment (start 147.683001 100.424999) (end 138.253002 90.995) (width 0.25) (layer B.Cu) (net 40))
 (segment (start 147.683001 107.674937) (end 147.683001 100.424999) (width 0.25) (layer B.Cu) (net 40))
 (segment (start 140.567937 114.790001) (end 147.683001 107.674937) (width 0.25) (layer B.Cu) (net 40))
 (segment (start 126.967999 114.790001) (end 140.567937 114.790001) (width 0.25) (layer B.Cu) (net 40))
 (segment (start 125.271669 113.093671) (end 126.967999 114.790001) (width 0.25) (layer B.Cu) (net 40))
 (segment (start 125.271669 91.967086) (end 125.271669 113.093671) (width 0.25) (layer B.Cu) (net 40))
 (segment (start 124.25567 90.951087) (end 125.271669 91.967086) (width 0.25) (layer B.Cu) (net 40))
 (segment (start 124.25567 89.981333) (end 124.25567 90.951087) (width 0.25) (layer B.Cu) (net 40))
 (segment (start 123.395085 85.487915) (end 124.730915 85.487915) (width 0.25) (layer B.Cu) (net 41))
 (segment (start 114.808 94.075) (end 123.395085 85.487915) (width 0.25) (layer B.Cu) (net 41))
 (segment (start 126.595329 91.967086) (end 126.920331 91.642084) (width 0.25) (layer F.Cu) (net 42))
 (segment (start 117.625086 91.967086) (end 126.595329 91.967086) (width 0.25) (layer F.Cu) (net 42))
 (segment (start 115.733 90.075) (end 117.625086 91.967086) (width 0.25) (layer F.Cu) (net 42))
 (segment (start 126.920331 91.642084) (end 127.52033 91.042085) (width 0.25) (layer F.Cu) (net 42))
 (segment (start 114.808 90.075) (end 115.733 90.075) (width 0.25) (layer F.Cu) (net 42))
 (segment (start 146.558 89.535) (end 151.638 84.455) (width 0.25) (layer B.Cu) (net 44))
 (segment (start 145.288 89.535) (end 146.558 89.535) (width 0.25) (layer B.Cu) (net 44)))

